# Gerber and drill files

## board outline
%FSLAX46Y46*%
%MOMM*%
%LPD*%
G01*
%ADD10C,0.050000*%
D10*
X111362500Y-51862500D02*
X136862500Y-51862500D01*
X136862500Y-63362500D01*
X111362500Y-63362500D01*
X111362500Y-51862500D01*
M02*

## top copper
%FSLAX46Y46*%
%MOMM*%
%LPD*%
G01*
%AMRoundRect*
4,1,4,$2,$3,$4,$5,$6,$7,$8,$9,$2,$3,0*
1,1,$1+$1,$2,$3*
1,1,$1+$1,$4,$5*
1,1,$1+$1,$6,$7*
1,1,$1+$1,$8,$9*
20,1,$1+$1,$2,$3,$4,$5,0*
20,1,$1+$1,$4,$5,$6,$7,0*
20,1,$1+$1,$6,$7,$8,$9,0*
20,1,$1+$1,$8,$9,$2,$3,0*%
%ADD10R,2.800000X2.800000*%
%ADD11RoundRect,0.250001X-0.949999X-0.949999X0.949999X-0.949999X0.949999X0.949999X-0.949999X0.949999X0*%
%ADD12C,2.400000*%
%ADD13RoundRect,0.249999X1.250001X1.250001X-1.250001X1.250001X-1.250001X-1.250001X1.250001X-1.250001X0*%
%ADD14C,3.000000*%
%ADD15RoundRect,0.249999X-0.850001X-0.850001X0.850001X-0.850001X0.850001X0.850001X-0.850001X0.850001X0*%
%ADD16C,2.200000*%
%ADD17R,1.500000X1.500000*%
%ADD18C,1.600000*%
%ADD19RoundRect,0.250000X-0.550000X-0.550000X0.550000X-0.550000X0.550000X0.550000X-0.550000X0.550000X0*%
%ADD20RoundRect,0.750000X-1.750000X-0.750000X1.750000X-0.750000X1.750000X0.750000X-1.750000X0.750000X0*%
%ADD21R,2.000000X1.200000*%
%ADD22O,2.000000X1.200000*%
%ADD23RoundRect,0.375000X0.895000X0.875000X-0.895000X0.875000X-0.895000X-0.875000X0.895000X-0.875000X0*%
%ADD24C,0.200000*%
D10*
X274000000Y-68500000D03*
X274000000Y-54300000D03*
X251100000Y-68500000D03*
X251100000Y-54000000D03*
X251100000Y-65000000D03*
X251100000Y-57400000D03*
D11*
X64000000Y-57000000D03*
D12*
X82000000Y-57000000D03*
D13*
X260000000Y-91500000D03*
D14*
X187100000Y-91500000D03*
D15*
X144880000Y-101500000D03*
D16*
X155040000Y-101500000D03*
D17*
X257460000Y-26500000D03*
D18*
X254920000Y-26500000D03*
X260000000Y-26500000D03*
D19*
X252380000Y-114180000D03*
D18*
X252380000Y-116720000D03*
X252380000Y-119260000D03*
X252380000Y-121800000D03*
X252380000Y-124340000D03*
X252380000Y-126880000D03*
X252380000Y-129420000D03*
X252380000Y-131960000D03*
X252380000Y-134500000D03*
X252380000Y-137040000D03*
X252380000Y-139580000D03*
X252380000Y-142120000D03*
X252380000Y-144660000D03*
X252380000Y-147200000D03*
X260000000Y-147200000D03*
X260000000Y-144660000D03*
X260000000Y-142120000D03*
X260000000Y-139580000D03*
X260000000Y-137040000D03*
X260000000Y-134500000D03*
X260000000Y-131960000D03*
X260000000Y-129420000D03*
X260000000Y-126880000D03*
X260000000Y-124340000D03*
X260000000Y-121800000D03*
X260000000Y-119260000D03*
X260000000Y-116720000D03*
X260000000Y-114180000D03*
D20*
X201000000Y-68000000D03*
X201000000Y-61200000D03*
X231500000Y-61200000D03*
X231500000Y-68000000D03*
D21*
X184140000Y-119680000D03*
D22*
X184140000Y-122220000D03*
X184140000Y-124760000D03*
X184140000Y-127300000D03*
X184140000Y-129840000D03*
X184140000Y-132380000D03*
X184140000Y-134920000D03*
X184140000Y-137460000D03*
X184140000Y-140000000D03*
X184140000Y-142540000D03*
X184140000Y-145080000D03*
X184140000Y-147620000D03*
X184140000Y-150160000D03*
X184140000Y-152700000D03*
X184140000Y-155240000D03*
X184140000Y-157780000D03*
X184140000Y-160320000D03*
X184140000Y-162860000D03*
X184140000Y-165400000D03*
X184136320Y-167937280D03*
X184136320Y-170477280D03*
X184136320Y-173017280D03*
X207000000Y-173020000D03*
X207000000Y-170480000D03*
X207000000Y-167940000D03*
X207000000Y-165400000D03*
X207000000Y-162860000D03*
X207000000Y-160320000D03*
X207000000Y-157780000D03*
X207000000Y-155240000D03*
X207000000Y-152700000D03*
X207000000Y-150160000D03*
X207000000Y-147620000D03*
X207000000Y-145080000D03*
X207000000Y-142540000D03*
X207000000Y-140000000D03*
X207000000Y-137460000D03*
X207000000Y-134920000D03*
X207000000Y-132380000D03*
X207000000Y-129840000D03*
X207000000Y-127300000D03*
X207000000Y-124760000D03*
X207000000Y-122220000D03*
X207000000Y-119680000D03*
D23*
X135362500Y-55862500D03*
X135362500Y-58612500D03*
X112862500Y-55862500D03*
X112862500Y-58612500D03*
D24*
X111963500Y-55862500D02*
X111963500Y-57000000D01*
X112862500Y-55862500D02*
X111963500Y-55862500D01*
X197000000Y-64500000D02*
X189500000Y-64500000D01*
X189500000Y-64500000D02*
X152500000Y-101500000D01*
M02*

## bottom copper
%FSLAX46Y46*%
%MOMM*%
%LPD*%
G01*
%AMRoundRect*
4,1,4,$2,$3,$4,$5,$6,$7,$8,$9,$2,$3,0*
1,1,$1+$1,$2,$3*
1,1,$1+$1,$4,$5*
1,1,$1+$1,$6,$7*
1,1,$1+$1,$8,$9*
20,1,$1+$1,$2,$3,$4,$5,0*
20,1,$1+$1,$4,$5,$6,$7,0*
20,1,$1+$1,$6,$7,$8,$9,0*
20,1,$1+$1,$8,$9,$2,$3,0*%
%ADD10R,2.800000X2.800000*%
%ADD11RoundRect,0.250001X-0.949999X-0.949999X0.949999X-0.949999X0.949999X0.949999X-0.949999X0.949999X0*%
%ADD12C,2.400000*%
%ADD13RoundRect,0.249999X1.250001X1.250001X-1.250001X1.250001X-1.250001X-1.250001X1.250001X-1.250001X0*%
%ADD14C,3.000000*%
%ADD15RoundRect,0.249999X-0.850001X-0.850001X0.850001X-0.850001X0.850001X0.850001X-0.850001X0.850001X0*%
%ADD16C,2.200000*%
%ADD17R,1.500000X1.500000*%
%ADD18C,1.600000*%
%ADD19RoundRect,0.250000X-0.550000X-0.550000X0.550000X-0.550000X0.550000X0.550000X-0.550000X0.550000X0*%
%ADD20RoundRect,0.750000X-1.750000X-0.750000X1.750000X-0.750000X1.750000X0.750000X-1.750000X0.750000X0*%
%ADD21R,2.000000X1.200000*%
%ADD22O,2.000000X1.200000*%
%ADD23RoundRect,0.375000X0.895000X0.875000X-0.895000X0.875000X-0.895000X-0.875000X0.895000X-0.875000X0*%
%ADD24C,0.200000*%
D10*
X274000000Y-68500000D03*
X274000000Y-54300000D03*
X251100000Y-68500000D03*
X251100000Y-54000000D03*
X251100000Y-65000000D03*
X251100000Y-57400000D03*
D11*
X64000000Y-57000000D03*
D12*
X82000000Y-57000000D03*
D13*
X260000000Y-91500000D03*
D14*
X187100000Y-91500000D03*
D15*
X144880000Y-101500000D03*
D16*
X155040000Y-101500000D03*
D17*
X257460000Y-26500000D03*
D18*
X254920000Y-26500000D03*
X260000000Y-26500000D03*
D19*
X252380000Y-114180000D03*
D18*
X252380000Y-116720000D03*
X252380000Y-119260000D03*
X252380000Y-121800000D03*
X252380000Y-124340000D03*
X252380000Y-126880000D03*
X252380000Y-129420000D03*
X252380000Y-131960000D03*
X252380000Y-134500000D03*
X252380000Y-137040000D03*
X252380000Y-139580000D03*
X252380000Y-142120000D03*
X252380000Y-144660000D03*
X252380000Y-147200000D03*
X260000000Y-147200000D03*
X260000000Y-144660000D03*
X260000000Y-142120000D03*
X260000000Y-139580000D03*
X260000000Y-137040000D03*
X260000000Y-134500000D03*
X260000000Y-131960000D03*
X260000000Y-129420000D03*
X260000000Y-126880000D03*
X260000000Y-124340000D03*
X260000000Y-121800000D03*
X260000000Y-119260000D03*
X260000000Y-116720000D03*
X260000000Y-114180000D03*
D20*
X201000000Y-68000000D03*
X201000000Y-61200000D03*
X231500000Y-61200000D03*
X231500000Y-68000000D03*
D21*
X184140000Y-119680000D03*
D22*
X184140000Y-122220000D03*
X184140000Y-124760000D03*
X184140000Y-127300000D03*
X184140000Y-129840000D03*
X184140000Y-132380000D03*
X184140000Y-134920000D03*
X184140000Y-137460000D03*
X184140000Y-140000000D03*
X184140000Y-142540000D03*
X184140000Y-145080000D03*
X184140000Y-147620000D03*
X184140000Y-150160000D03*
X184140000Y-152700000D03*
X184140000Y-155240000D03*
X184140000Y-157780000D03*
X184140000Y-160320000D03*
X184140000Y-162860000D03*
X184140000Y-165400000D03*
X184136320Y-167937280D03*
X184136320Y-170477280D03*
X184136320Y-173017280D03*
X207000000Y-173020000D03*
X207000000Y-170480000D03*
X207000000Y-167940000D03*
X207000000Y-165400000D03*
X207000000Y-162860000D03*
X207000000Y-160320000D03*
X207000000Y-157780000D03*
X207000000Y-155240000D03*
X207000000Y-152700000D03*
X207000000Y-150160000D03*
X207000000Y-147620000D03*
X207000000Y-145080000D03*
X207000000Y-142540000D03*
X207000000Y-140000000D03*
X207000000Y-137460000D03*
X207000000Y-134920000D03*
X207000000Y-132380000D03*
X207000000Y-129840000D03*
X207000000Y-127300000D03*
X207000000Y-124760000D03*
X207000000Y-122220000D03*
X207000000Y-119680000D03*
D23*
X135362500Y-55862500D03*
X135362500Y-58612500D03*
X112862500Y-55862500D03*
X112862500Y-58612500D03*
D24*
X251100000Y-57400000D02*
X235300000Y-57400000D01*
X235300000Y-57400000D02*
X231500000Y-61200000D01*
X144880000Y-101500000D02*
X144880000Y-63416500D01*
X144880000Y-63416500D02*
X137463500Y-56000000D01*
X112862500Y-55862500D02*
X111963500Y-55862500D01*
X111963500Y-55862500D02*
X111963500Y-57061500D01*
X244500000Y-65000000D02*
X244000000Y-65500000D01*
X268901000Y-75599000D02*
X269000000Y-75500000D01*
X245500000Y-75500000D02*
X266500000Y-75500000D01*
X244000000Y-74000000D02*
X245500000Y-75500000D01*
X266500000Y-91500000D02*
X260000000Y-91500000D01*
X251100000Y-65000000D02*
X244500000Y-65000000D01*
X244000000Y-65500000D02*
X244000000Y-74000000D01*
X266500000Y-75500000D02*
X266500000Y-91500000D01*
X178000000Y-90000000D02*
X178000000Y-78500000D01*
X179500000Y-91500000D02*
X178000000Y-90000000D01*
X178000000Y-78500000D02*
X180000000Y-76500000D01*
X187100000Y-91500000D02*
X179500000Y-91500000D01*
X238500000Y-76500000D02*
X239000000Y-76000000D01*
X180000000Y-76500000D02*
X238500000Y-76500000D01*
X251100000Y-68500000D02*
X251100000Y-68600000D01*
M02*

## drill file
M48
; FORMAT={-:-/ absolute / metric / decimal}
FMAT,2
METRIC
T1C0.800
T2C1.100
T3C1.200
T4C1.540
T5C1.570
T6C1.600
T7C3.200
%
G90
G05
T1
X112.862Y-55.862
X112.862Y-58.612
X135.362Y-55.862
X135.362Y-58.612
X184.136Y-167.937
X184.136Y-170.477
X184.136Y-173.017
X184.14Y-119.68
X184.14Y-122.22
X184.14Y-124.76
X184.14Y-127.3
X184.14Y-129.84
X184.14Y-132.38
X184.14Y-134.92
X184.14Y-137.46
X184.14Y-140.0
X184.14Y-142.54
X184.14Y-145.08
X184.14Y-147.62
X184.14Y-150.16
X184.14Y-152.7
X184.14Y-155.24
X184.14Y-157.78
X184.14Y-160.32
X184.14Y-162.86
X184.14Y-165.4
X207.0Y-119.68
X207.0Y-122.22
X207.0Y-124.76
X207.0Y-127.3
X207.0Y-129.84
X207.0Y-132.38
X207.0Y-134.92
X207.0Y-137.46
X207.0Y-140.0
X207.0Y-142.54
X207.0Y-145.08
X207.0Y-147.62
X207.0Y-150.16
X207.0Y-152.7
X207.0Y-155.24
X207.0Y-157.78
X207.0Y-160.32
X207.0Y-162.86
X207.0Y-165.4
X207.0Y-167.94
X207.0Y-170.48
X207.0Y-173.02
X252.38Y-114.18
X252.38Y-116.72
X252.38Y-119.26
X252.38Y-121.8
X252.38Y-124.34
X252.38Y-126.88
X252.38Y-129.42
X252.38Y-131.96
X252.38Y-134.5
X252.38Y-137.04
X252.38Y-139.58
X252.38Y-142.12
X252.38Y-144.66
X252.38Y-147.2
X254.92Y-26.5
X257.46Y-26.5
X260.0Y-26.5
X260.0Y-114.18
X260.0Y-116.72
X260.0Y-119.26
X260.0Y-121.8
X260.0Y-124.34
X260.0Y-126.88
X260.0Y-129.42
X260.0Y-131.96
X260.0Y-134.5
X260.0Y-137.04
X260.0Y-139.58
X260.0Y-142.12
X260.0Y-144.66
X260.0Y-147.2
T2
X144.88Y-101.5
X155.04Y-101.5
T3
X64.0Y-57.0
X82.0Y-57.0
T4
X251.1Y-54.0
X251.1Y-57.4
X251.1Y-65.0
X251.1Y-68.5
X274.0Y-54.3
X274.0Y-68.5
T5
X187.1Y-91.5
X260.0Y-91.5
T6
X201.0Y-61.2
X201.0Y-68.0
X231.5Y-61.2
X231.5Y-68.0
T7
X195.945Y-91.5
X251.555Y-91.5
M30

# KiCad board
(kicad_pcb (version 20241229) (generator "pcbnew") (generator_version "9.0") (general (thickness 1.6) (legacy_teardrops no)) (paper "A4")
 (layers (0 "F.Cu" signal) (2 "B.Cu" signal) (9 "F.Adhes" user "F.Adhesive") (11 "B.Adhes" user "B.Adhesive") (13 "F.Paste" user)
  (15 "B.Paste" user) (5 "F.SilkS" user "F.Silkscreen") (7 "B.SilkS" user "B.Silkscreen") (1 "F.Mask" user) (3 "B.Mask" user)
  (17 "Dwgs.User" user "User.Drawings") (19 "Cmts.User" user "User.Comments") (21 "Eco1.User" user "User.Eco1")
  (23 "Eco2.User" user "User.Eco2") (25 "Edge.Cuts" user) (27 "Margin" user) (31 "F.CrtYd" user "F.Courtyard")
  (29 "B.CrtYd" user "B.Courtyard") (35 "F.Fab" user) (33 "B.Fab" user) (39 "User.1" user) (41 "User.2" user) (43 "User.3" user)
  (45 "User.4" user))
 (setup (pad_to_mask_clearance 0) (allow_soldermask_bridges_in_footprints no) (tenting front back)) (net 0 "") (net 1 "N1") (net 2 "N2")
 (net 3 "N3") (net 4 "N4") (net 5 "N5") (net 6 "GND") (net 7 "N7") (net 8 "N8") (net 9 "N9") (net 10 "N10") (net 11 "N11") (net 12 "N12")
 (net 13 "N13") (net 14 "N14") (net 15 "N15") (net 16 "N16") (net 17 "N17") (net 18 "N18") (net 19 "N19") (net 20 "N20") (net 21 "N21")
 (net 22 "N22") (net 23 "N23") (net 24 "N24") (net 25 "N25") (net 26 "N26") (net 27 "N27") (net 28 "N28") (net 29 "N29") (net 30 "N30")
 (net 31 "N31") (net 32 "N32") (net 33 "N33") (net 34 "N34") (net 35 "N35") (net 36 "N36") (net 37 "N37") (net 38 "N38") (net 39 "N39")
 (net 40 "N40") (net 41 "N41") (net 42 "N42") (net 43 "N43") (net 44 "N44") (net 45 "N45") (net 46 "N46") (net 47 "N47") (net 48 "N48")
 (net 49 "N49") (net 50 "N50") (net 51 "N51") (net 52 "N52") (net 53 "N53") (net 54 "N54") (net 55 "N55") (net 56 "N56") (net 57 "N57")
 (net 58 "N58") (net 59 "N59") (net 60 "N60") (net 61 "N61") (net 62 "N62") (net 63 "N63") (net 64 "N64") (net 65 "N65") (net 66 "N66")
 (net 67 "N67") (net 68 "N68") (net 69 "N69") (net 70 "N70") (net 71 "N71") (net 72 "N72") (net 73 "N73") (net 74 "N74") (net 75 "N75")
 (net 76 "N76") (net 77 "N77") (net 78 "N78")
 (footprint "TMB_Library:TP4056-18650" (layer "F.Cu") (at 275.7 70.2 180)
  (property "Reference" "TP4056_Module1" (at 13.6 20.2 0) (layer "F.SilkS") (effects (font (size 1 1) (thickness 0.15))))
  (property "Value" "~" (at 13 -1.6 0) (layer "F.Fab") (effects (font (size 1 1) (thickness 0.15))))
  (pad "1" thru_hole rect (at 1.7 1.7 180) (size 2.8 2.8) (drill 1.54) (layers "*.Cu" "*.Mask") (remove_unused_layers no) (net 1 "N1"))
  (pad "2" thru_hole rect (at 1.7 15.9 180) (size 2.8 2.8) (drill 1.54) (layers "*.Cu" "*.Mask") (remove_unused_layers no) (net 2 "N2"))
  (pad "3" thru_hole rect (at 24.6 1.7 180) (size 2.8 2.8) (drill 1.54) (layers "*.Cu" "*.Mask") (remove_unused_layers no) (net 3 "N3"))
  (pad "4" thru_hole rect (at 24.6 16.2 180) (size 2.8 2.8) (drill 1.54) (layers "*.Cu" "*.Mask") (remove_unused_layers no) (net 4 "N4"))
  (pad "5" thru_hole rect (at 24.6 5.2 180) (size 2.8 2.8) (drill 1.54) (layers "*.Cu" "*.Mask") (remove_unused_layers no) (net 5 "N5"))
  (pad "6" thru_hole rect (at 24.6 12.8 180) (size 2.8 2.8) (drill 1.54) (layers "*.Cu" "*.Mask") (remove_unused_layers no) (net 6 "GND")))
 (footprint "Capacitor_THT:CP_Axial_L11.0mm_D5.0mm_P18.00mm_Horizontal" (layer "F.Cu") (at 64 57)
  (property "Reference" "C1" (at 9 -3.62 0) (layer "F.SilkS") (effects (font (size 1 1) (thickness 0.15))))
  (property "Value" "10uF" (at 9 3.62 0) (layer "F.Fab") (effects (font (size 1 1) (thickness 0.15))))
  (pad "1" thru_hole roundrect (at 0 0) (size 2.4 2.4) (drill 1.2) (layers "*.Cu" "*.Mask") (remove_unused_layers no)
   (roundrect_rratio 0.104167) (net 6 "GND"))
  (pad "2" thru_hole circle (at 18 0) (size 2.4 2.4) (drill 1.2) (layers "*.Cu" "*.Mask") (remove_unused_layers no) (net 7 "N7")))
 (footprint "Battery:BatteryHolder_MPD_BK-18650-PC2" (layer "F.Cu") (at 260 91.5 180)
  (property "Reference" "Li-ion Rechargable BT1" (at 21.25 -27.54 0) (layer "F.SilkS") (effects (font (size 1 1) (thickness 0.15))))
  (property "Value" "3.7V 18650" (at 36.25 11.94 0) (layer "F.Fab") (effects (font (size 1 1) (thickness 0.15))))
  (pad "" np_thru_hole circle (at 8.445 0 180) (size 3.2 3.2) (drill 3.2) (layers "*.Cu" "*.Mask"))
  (pad "" np_thru_hole circle (at 64.055 0 180) (size 3.2 3.2) (drill 3.2) (layers "*.Cu" "*.Mask"))
  (pad "1" thru_hole roundrect (at 0 0 180) (size 3 3) (drill 1.57) (layers "*.Cu" "*.Mask") (remove_unused_layers no)
   (roundrect_rratio 0.083333) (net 5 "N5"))
  (pad "2" thru_hole circle (at 72.9 0 180) (size 3 3) (drill 1.57) (layers "*.Cu" "*.Mask") (remove_unused_layers no) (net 4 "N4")))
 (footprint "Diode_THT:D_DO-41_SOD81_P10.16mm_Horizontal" (layer "F.Cu") (at 144.88 101.5)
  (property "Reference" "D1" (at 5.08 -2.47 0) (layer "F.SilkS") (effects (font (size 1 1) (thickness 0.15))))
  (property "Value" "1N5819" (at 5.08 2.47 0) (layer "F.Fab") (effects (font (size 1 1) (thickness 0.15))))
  (pad "1" thru_hole roundrect (at 0 0) (size 2.2 2.2) (drill 1.1) (layers "*.Cu" "*.Mask") (remove_unused_layers no)
   (roundrect_rratio 0.113636) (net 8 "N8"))
  (pad "2" thru_hole circle (at 10.16 0) (size 2.2 2.2) (drill 1.1) (layers "*.Cu" "*.Mask") (remove_unused_layers no) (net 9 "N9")))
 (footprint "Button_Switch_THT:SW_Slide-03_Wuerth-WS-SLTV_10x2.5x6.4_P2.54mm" (layer "F.Cu") (at 257.46 26.5)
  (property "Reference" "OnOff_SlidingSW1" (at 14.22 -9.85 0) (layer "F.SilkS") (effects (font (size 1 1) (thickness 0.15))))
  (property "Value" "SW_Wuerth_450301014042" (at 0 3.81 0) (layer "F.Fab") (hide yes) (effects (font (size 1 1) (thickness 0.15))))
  (pad "1" thru_hole rect (at 0 0) (size 1.5 1.5) (drill 0.8) (layers "*.Cu" "*.Mask") (remove_unused_layers no) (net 3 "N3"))
  (pad "2" thru_hole circle (at -2.54 0) (size 1.6 1.6) (drill 0.8) (layers "*.Cu" "*.Mask") (remove_unused_layers no) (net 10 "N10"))
  (pad "3" thru_hole circle (at 2.54 0) (size 1.6 1.6) (drill 0.8) (layers "*.Cu" "*.Mask") (remove_unused_layers no) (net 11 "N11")))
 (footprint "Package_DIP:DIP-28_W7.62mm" (layer "F.Cu") (at 252.38 114.18)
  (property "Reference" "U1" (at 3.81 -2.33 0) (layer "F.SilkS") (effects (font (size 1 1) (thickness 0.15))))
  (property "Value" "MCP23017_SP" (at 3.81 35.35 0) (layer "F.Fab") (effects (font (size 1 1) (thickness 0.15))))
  (pad "1" thru_hole roundrect (at 0 0) (size 1.6 1.6) (drill 0.8) (layers "*.Cu" "*.Mask") (remove_unused_layers no)
   (roundrect_rratio 0.15625) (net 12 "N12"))
  (pad "2" thru_hole circle (at 0 2.54) (size 1.6 1.6) (drill 0.8) (layers "*.Cu" "*.Mask") (remove_unused_layers no) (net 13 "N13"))
  (pad "3" thru_hole circle (at 0 5.08) (size 1.6 1.6) (drill 0.8) (layers "*.Cu" "*.Mask") (remove_unused_layers no) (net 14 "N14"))
  (pad "4" thru_hole circle (at 0 7.62) (size 1.6 1.6) (drill 0.8) (layers "*.Cu" "*.Mask") (remove_unused_layers no) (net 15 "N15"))
  (pad "5" thru_hole circle (at 0 10.16) (size 1.6 1.6) (drill 0.8) (layers "*.Cu" "*.Mask") (remove_unused_layers no) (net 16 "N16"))
  (pad "6" thru_hole circle (at 0 12.7) (size 1.6 1.6) (drill 0.8) (layers "*.Cu" "*.Mask") (remove_unused_layers no) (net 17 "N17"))
  (pad "7" thru_hole circle (at 0 15.24) (size 1.6 1.6) (drill 0.8) (layers "*.Cu" "*.Mask") (remove_unused_layers no) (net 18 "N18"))
  (pad "8" thru_hole circle (at 0 17.78) (size 1.6 1.6) (drill 0.8) (layers "*.Cu" "*.Mask") (remove_unused_layers no) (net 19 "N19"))
  (pad "9" thru_hole circle (at 0 20.32) (size 1.6 1.6) (drill 0.8) (layers "*.Cu" "*.Mask") (remove_unused_layers no) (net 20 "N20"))
  (pad "10" thru_hole circle (at 0 22.86) (size 1.6 1.6) (drill 0.8) (layers "*.Cu" "*.Mask") (remove_unused_layers no) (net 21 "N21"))
  (pad "11" thru_hole circle (at 0 25.4) (size 1.6 1.6) (drill 0.8) (layers "*.Cu" "*.Mask") (remove_unused_layers no) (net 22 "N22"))
  (pad "12" thru_hole circle (at 0 27.94) (size 1.6 1.6) (drill 0.8) (layers "*.Cu" "*.Mask") (remove_unused_layers no) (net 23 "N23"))
  (pad "13" thru_hole circle (at 0 30.48) (size 1.6 1.6) (drill 0.8) (layers "*.Cu" "*.Mask") (remove_unused_layers no) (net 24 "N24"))
  (pad "14" thru_hole circle (at 0 33.02) (size 1.6 1.6) (drill 0.8) (layers "*.Cu" "*.Mask") (remove_unused_layers no) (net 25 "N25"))
  (pad "15" thru_hole circle (at 7.62 33.02) (size 1.6 1.6) (drill 0.8) (layers "*.Cu" "*.Mask") (remove_unused_layers no) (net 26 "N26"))
  (pad "16" thru_hole circle (at 7.62 30.48) (size 1.6 1.6) (drill 0.8) (layers "*.Cu" "*.Mask") (remove_unused_layers no) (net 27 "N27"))
  (pad "17" thru_hole circle (at 7.62 27.94) (size 1.6 1.6) (drill 0.8) (layers "*.Cu" "*.Mask") (remove_unused_layers no) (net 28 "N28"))
  (pad "18" thru_hole circle (at 7.62 25.4) (size 1.6 1.6) (drill 0.8) (layers "*.Cu" "*.Mask") (remove_unused_layers no) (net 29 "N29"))
  (pad "19" thru_hole circle (at 7.62 22.86) (size 1.6 1.6) (drill 0.8) (layers "*.Cu" "*.Mask") (remove_unused_layers no) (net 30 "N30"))
  (pad "20" thru_hole circle (at 7.62 20.32) (size 1.6 1.6) (drill 0.8) (layers "*.Cu" "*.Mask") (remove_unused_layers no) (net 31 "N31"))
  (pad "21" thru_hole circle (at 7.62 17.78) (size 1.6 1.6) (drill 0.8) (layers "*.Cu" "*.Mask") (remove_unused_layers no) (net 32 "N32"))
  (pad "22" thru_hole circle (at 7.62 15.24) (size 1.6 1.6) (drill 0.8) (layers "*.Cu" "*.Mask") (remove_unused_layers no) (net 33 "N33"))
  (pad "23" thru_hole circle (at 7.62 12.7) (size 1.6 1.6) (drill 0.8) (layers "*.Cu" "*.Mask") (remove_unused_layers no) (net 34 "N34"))
  (pad "24" thru_hole circle (at 7.62 10.16) (size 1.6 1.6) (drill 0.8) (layers "*.Cu" "*.Mask") (remove_unused_layers no) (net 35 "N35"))
  (pad "25" thru_hole circle (at 7.62 7.62) (size 1.6 1.6) (drill 0.8) (layers "*.Cu" "*.Mask") (remove_unused_layers no) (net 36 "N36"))
  (pad "26" thru_hole circle (at 7.62 5.08) (size 1.6 1.6) (drill 0.8) (layers "*.Cu" "*.Mask") (remove_unused_layers no) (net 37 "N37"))
  (pad "27" thru_hole circle (at 7.62 2.54) (size 1.6 1.6) (drill 0.8) (layers "*.Cu" "*.Mask") (remove_unused_layers no) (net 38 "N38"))
  (pad "28" thru_hole circle (at 7.62 0) (size 1.6 1.6) (drill 0.8) (layers "*.Cu" "*.Mask") (remove_unused_layers no) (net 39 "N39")))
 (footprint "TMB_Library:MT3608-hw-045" (layer "F.Cu") (at 216 65.1)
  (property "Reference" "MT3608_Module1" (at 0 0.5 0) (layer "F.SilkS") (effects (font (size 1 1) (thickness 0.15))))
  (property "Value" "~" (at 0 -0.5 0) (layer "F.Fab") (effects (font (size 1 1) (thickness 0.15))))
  (pad "1" thru_hole roundrect (at -15 2.9) (size 5 3) (drill 1.6) (layers "*.Cu" "*.Mask") (remove_unused_layers no)
   (roundrect_rratio 0.25) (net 10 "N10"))
  (pad "2" thru_hole roundrect (at -15 -3.9) (size 5 3) (drill 1.6) (layers "*.Cu" "*.Mask") (remove_unused_layers no)
   (roundrect_rratio 0.25) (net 6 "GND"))
  (pad "3" thru_hole roundrect (at 15.5 -3.9) (size 5 3) (drill 1.6) (layers "*.Cu" "*.Mask") (remove_unused_layers no)
   (roundrect_rratio 0.25) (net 6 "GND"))
  (pad "4" thru_hole roundrect (at 15.5 2.9) (size 5 3) (drill 1.6) (layers "*.Cu" "*.Mask") (remove_unused_layers no)
   (roundrect_rratio 0.25) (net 9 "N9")))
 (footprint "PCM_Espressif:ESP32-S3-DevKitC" (layer "F.Cu") (at 184.14 119.68)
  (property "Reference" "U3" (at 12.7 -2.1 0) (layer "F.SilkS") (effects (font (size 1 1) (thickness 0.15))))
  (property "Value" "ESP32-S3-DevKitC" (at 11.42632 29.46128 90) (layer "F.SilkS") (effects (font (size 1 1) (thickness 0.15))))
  (pad "1" thru_hole rect (at 0 0 270) (size 1.2 2) (drill 0.8) (layers "*.Cu" "*.Mask") (remove_unused_layers no) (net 7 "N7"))
  (pad "2" thru_hole oval (at 0 2.54 270) (size 1.2 2) (drill 0.8) (layers "*.Cu" "*.Mask") (remove_unused_layers no) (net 7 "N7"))
  (pad "3" thru_hole oval (at 0 5.08 270) (size 1.2 2) (drill 0.8) (layers "*.Cu" "*.Mask") (remove_unused_layers no) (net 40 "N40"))
  (pad "4" thru_hole oval (at 0 7.62 270) (size 1.2 2) (drill 0.8) (layers "*.Cu" "*.Mask") (remove_unused_layers no) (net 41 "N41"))
  (pad "5" thru_hole oval (at 0 10.16 270) (size 1.2 2) (drill 0.8) (layers "*.Cu" "*.Mask") (remove_unused_layers no) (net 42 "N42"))
  (pad "6" thru_hole oval (at 0 12.7 270) (size 1.2 2) (drill 0.8) (layers "*.Cu" "*.Mask") (remove_unused_layers no) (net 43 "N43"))
  (pad "7" thru_hole oval (at 0 15.24 270) (size 1.2 2) (drill 0.8) (layers "*.Cu" "*.Mask") (remove_unused_layers no) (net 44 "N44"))
  (pad "8" thru_hole oval (at 0 17.78 270) (size 1.2 2) (drill 0.8) (layers "*.Cu" "*.Mask") (remove_unused_layers no) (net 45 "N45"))
  (pad "9" thru_hole oval (at 0 20.32 270) (size 1.2 2) (drill 0.8) (layers "*.Cu" "*.Mask") (remove_unused_layers no) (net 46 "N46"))
  (pad "10" thru_hole oval (at 0 22.86 270) (size 1.2 2) (drill 0.8) (layers "*.Cu" "*.Mask") (remove_unused_layers no) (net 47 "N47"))
  (pad "11" thru_hole oval (at 0 25.4 270) (size 1.2 2) (drill 0.8) (layers "*.Cu" "*.Mask") (remove_unused_layers no) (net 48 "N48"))
  (pad "12" thru_hole oval (at 0 27.94 270) (size 1.2 2) (drill 0.8) (layers "*.Cu" "*.Mask") (remove_unused_layers no) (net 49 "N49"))
  (pad "13" thru_hole oval (at 0 30.48 270) (size 1.2 2) (drill 0.8) (layers "*.Cu" "*.Mask") (remove_unused_layers no) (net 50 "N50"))
  (pad "14" thru_hole oval (at 0 33.02 270) (size 1.2 2) (drill 0.8) (layers "*.Cu" "*.Mask") (remove_unused_layers no) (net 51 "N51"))
  (pad "15" thru_hole oval (at 0 35.56 270) (size 1.2 2) (drill 0.8) (layers "*.Cu" "*.Mask") (remove_unused_layers no) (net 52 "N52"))
  (pad "16" thru_hole oval (at 0 38.1 270) (size 1.2 2) (drill 0.8) (layers "*.Cu" "*.Mask") (remove_unused_layers no) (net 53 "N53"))
  (pad "17" thru_hole oval (at 0 40.64 270) (size 1.2 2) (drill 0.8) (layers "*.Cu" "*.Mask") (remove_unused_layers no) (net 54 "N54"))
  (pad "18" thru_hole oval (at 0 43.18 270) (size 1.2 2) (drill 0.8) (layers "*.Cu" "*.Mask") (remove_unused_layers no) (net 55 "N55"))
  (pad "19" thru_hole oval (at 0 45.72 270) (size 1.2 2) (drill 0.8) (layers "*.Cu" "*.Mask") (remove_unused_layers no) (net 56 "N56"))
  (pad "20" thru_hole oval (at -0.00368 48.25728 270) (size 1.2 2) (drill 0.8) (layers "*.Cu" "*.Mask") (remove_unused_layers no)
   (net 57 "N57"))
  (pad "21" thru_hole oval (at -0.00368 50.79728 270) (size 1.2 2) (drill 0.8) (layers "*.Cu" "*.Mask") (remove_unused_layers no)
   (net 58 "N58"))
  (pad "22" thru_hole oval (at -0.00368 53.33728 270) (size 1.2 2) (drill 0.8) (layers "*.Cu" "*.Mask") (remove_unused_layers no)
   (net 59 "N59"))
  (pad "23" thru_hole oval (at 22.86 53.34 270) (size 1.2 2) (drill 0.8) (layers "*.Cu" "*.Mask") (remove_unused_layers no) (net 59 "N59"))
  (pad "24" thru_hole oval (at 22.86 50.8 270) (size 1.2 2) (drill 0.8) (layers "*.Cu" "*.Mask") (remove_unused_layers no) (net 59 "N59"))
  (pad "25" thru_hole oval (at 22.86 48.26 270) (size 1.2 2) (drill 0.8) (layers "*.Cu" "*.Mask") (remove_unused_layers no) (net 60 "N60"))
  (pad "26" thru_hole oval (at 22.86 45.72 270) (size 1.2 2) (drill 0.8) (layers "*.Cu" "*.Mask") (remove_unused_layers no) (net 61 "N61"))
  (pad "27" thru_hole oval (at 22.86 43.18 270) (size 1.2 2) (drill 0.8) (layers "*.Cu" "*.Mask") (remove_unused_layers no) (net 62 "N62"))
  (pad "28" thru_hole oval (at 22.86 40.64 270) (size 1.2 2) (drill 0.8) (layers "*.Cu" "*.Mask") (remove_unused_layers no) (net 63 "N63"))
  (pad "29" thru_hole oval (at 22.86 38.1 270) (size 1.2 2) (drill 0.8) (layers "*.Cu" "*.Mask") (remove_unused_layers no) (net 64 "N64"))
  (pad "30" thru_hole oval (at 22.86 35.56 270) (size 1.2 2) (drill 0.8) (layers "*.Cu" "*.Mask") (remove_unused_layers no) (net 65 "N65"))
  (pad "31" thru_hole oval (at 22.86 33.02 270) (size 1.2 2) (drill 0.8) (layers "*.Cu" "*.Mask") (remove_unused_layers no) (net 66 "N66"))
  (pad "32" thru_hole oval (at 22.86 30.48 270) (size 1.2 2) (drill 0.8) (layers "*.Cu" "*.Mask") (remove_unused_layers no) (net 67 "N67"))
  (pad "33" thru_hole oval (at 22.86 27.94 270) (size 1.2 2) (drill 0.8) (layers "*.Cu" "*.Mask") (remove_unused_layers no) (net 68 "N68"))
  (pad "34" thru_hole oval (at 22.86 25.4 270) (size 1.2 2) (drill 0.8) (layers "*.Cu" "*.Mask") (remove_unused_layers no) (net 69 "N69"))
  (pad "35" thru_hole oval (at 22.86 22.86 270) (size 1.2 2) (drill 0.8) (layers "*.Cu" "*.Mask") (remove_unused_layers no) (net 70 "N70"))
  (pad "36" thru_hole oval (at 22.86 20.32 270) (size 1.2 2) (drill 0.8) (layers "*.Cu" "*.Mask") (remove_unused_layers no) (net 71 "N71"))
  (pad "37" thru_hole oval (at 22.86 17.78 270) (size 1.2 2) (drill 0.8) (layers "*.Cu" "*.Mask") (remove_unused_layers no) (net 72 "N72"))
  (pad "38" thru_hole oval (at 22.86 15.24 270) (size 1.2 2) (drill 0.8) (layers "*.Cu" "*.Mask") (remove_unused_layers no) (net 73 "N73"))
  (pad "39" thru_hole oval (at 22.86 12.7 270) (size 1.2 2) (drill 0.8) (layers "*.Cu" "*.Mask") (remove_unused_layers no) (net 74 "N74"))
  (pad "40" thru_hole oval (at 22.86 10.16 270) (size 1.2 2) (drill 0.8) (layers "*.Cu" "*.Mask") (remove_unused_layers no) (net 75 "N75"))
  (pad "41" thru_hole oval (at 22.86 7.62 270) (size 1.2 2) (drill 0.8) (layers "*.Cu" "*.Mask") (remove_unused_layers no) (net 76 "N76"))
  (pad "42" thru_hole oval (at 22.86 5.08 270) (size 1.2 2) (drill 0.8) (layers "*.Cu" "*.Mask") (remove_unused_layers no) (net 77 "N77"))
  (pad "43" thru_hole oval (at 22.86 2.54 270) (size 1.2 2) (drill 0.8) (layers "*.Cu" "*.Mask") (remove_unused_layers no) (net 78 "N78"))
  (pad "44" thru_hole oval (at 22.86 0 270) (size 1.2 2) (drill 0.8) (layers "*.Cu" "*.Mask") (remove_unused_layers no) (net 59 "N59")))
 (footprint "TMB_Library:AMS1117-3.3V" (layer "F.Cu") (at 111.3625 51.8625)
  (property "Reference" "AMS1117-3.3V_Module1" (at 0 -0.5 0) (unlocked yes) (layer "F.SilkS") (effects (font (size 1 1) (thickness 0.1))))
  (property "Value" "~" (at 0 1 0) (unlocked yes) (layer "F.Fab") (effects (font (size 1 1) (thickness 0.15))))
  (fp_rect (start 0 0) (end 25.5 11.5) (stroke (width 0.05) (type solid)) (fill no) (layer "Edge.Cuts"))
  (pad "1" thru_hole roundrect (at 24 4 180) (size 2.54 2.5) (drill 0.8) (layers "*.Cu" "*.Mask") (remove_unused_layers no)
   (roundrect_rratio 0.15) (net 8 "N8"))
  (pad "2" thru_hole roundrect (at 24 6.75 180) (size 2.54 2.5) (drill 0.8) (layers "*.Cu" "*.Mask") (remove_unused_layers no)
   (roundrect_rratio 0.15) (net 6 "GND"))
  (pad "3" thru_hole roundrect (at 1.5 4 180) (size 2.54 2.5) (drill 0.8) (layers "*.Cu" "*.Mask") (remove_unused_layers no)
   (roundrect_rratio 0.15) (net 7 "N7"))
  (pad "4" thru_hole roundrect (at 1.5 6.75 180) (size 2.54 2.5) (drill 0.8) (layers "*.Cu" "*.Mask") (remove_unused_layers no)
   (roundrect_rratio 0.15) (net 6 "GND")))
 (segment (start 251.1 57.4) (end 235.3 57.4) (width 0.2) (layer "B.Cu") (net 6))
 (segment (start 235.3 57.4) (end 231.5 61.2) (width 0.2) (layer "B.Cu") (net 6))
 (segment (start 144.88 101.5) (end 144.88 63.4165) (width 0.2) (layer "B.Cu") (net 8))
 (segment (start 144.88 63.4165) (end 137.4635 56) (width 0.2) (layer "B.Cu") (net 8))
 (segment (start 111.9635 55.8625) (end 111.9635 57) (width 0.2) (layer "F.Cu") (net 7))
 (segment (start 112.8625 55.8625) (end 111.9635 55.8625) (width 0.2) (layer "F.Cu") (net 7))
 (segment (start 112.8625 55.8625) (end 111.9635 55.8625) (width 0.2) (layer "B.Cu") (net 7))
 (segment (start 111.9635 55.8625) (end 111.9635 57.0615) (width 0.2) (layer "B.Cu") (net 7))
 (segment (start 197 64.5) (end 189.5 64.5) (width 0.2) (layer "F.Cu") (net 9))
 (segment (start 189.5 64.5) (end 152.5 101.5) (width 0.2) (layer "F.Cu") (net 9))
 (segment (start 244.5 65) (end 244 65.5) (width 0.2) (layer "B.Cu") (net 5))
 (segment (start 268.901 75.599) (end 269 75.5) (width 0.2) (layer "B.Cu") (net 5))
 (segment (start 245.5 75.5) (end 266.5 75.5) (width 0.2) (layer "B.Cu") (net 5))
 (segment (start 244 74) (end 245.5 75.5) (width 0.2) (layer "B.Cu") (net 5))
 (segment (start 266.5 91.5) (end 260 91.5) (width 0.2) (layer "B.Cu") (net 5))
 (segment (start 251.1 65) (end 244.5 65) (width 0.2) (layer "B.Cu") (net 5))
 (segment (start 244 65.5) (end 244 74) (width 0.2) (layer "B.Cu") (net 5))
 (segment (start 266.5 75.5) (end 266.5 91.5) (width 0.2) (layer "B.Cu") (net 5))
 (segment (start 178 90) (end 178 78.5) (width 0.2) (layer "B.Cu") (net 4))
 (segment (start 179.5 91.5) (end 178 90) (width 0.2) (layer "B.Cu") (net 4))
 (segment (start 178 78.5) (end 180 76.5) (width 0.2) (layer "B.Cu") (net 4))
 (segment (start 187.1 91.5) (end 179.5 91.5) (width 0.2) (layer "B.Cu") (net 4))
 (segment (start 238.5 76.5) (end 239 76) (width 0.2) (layer "B.Cu") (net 4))
 (segment (start 180 76.5) (end 238.5 76.5) (width 0.2) (layer "B.Cu") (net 4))
 (segment (start 251.1 68.5) (end 251.1 68.6) (width 0.2) (layer "B.Cu") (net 3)))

